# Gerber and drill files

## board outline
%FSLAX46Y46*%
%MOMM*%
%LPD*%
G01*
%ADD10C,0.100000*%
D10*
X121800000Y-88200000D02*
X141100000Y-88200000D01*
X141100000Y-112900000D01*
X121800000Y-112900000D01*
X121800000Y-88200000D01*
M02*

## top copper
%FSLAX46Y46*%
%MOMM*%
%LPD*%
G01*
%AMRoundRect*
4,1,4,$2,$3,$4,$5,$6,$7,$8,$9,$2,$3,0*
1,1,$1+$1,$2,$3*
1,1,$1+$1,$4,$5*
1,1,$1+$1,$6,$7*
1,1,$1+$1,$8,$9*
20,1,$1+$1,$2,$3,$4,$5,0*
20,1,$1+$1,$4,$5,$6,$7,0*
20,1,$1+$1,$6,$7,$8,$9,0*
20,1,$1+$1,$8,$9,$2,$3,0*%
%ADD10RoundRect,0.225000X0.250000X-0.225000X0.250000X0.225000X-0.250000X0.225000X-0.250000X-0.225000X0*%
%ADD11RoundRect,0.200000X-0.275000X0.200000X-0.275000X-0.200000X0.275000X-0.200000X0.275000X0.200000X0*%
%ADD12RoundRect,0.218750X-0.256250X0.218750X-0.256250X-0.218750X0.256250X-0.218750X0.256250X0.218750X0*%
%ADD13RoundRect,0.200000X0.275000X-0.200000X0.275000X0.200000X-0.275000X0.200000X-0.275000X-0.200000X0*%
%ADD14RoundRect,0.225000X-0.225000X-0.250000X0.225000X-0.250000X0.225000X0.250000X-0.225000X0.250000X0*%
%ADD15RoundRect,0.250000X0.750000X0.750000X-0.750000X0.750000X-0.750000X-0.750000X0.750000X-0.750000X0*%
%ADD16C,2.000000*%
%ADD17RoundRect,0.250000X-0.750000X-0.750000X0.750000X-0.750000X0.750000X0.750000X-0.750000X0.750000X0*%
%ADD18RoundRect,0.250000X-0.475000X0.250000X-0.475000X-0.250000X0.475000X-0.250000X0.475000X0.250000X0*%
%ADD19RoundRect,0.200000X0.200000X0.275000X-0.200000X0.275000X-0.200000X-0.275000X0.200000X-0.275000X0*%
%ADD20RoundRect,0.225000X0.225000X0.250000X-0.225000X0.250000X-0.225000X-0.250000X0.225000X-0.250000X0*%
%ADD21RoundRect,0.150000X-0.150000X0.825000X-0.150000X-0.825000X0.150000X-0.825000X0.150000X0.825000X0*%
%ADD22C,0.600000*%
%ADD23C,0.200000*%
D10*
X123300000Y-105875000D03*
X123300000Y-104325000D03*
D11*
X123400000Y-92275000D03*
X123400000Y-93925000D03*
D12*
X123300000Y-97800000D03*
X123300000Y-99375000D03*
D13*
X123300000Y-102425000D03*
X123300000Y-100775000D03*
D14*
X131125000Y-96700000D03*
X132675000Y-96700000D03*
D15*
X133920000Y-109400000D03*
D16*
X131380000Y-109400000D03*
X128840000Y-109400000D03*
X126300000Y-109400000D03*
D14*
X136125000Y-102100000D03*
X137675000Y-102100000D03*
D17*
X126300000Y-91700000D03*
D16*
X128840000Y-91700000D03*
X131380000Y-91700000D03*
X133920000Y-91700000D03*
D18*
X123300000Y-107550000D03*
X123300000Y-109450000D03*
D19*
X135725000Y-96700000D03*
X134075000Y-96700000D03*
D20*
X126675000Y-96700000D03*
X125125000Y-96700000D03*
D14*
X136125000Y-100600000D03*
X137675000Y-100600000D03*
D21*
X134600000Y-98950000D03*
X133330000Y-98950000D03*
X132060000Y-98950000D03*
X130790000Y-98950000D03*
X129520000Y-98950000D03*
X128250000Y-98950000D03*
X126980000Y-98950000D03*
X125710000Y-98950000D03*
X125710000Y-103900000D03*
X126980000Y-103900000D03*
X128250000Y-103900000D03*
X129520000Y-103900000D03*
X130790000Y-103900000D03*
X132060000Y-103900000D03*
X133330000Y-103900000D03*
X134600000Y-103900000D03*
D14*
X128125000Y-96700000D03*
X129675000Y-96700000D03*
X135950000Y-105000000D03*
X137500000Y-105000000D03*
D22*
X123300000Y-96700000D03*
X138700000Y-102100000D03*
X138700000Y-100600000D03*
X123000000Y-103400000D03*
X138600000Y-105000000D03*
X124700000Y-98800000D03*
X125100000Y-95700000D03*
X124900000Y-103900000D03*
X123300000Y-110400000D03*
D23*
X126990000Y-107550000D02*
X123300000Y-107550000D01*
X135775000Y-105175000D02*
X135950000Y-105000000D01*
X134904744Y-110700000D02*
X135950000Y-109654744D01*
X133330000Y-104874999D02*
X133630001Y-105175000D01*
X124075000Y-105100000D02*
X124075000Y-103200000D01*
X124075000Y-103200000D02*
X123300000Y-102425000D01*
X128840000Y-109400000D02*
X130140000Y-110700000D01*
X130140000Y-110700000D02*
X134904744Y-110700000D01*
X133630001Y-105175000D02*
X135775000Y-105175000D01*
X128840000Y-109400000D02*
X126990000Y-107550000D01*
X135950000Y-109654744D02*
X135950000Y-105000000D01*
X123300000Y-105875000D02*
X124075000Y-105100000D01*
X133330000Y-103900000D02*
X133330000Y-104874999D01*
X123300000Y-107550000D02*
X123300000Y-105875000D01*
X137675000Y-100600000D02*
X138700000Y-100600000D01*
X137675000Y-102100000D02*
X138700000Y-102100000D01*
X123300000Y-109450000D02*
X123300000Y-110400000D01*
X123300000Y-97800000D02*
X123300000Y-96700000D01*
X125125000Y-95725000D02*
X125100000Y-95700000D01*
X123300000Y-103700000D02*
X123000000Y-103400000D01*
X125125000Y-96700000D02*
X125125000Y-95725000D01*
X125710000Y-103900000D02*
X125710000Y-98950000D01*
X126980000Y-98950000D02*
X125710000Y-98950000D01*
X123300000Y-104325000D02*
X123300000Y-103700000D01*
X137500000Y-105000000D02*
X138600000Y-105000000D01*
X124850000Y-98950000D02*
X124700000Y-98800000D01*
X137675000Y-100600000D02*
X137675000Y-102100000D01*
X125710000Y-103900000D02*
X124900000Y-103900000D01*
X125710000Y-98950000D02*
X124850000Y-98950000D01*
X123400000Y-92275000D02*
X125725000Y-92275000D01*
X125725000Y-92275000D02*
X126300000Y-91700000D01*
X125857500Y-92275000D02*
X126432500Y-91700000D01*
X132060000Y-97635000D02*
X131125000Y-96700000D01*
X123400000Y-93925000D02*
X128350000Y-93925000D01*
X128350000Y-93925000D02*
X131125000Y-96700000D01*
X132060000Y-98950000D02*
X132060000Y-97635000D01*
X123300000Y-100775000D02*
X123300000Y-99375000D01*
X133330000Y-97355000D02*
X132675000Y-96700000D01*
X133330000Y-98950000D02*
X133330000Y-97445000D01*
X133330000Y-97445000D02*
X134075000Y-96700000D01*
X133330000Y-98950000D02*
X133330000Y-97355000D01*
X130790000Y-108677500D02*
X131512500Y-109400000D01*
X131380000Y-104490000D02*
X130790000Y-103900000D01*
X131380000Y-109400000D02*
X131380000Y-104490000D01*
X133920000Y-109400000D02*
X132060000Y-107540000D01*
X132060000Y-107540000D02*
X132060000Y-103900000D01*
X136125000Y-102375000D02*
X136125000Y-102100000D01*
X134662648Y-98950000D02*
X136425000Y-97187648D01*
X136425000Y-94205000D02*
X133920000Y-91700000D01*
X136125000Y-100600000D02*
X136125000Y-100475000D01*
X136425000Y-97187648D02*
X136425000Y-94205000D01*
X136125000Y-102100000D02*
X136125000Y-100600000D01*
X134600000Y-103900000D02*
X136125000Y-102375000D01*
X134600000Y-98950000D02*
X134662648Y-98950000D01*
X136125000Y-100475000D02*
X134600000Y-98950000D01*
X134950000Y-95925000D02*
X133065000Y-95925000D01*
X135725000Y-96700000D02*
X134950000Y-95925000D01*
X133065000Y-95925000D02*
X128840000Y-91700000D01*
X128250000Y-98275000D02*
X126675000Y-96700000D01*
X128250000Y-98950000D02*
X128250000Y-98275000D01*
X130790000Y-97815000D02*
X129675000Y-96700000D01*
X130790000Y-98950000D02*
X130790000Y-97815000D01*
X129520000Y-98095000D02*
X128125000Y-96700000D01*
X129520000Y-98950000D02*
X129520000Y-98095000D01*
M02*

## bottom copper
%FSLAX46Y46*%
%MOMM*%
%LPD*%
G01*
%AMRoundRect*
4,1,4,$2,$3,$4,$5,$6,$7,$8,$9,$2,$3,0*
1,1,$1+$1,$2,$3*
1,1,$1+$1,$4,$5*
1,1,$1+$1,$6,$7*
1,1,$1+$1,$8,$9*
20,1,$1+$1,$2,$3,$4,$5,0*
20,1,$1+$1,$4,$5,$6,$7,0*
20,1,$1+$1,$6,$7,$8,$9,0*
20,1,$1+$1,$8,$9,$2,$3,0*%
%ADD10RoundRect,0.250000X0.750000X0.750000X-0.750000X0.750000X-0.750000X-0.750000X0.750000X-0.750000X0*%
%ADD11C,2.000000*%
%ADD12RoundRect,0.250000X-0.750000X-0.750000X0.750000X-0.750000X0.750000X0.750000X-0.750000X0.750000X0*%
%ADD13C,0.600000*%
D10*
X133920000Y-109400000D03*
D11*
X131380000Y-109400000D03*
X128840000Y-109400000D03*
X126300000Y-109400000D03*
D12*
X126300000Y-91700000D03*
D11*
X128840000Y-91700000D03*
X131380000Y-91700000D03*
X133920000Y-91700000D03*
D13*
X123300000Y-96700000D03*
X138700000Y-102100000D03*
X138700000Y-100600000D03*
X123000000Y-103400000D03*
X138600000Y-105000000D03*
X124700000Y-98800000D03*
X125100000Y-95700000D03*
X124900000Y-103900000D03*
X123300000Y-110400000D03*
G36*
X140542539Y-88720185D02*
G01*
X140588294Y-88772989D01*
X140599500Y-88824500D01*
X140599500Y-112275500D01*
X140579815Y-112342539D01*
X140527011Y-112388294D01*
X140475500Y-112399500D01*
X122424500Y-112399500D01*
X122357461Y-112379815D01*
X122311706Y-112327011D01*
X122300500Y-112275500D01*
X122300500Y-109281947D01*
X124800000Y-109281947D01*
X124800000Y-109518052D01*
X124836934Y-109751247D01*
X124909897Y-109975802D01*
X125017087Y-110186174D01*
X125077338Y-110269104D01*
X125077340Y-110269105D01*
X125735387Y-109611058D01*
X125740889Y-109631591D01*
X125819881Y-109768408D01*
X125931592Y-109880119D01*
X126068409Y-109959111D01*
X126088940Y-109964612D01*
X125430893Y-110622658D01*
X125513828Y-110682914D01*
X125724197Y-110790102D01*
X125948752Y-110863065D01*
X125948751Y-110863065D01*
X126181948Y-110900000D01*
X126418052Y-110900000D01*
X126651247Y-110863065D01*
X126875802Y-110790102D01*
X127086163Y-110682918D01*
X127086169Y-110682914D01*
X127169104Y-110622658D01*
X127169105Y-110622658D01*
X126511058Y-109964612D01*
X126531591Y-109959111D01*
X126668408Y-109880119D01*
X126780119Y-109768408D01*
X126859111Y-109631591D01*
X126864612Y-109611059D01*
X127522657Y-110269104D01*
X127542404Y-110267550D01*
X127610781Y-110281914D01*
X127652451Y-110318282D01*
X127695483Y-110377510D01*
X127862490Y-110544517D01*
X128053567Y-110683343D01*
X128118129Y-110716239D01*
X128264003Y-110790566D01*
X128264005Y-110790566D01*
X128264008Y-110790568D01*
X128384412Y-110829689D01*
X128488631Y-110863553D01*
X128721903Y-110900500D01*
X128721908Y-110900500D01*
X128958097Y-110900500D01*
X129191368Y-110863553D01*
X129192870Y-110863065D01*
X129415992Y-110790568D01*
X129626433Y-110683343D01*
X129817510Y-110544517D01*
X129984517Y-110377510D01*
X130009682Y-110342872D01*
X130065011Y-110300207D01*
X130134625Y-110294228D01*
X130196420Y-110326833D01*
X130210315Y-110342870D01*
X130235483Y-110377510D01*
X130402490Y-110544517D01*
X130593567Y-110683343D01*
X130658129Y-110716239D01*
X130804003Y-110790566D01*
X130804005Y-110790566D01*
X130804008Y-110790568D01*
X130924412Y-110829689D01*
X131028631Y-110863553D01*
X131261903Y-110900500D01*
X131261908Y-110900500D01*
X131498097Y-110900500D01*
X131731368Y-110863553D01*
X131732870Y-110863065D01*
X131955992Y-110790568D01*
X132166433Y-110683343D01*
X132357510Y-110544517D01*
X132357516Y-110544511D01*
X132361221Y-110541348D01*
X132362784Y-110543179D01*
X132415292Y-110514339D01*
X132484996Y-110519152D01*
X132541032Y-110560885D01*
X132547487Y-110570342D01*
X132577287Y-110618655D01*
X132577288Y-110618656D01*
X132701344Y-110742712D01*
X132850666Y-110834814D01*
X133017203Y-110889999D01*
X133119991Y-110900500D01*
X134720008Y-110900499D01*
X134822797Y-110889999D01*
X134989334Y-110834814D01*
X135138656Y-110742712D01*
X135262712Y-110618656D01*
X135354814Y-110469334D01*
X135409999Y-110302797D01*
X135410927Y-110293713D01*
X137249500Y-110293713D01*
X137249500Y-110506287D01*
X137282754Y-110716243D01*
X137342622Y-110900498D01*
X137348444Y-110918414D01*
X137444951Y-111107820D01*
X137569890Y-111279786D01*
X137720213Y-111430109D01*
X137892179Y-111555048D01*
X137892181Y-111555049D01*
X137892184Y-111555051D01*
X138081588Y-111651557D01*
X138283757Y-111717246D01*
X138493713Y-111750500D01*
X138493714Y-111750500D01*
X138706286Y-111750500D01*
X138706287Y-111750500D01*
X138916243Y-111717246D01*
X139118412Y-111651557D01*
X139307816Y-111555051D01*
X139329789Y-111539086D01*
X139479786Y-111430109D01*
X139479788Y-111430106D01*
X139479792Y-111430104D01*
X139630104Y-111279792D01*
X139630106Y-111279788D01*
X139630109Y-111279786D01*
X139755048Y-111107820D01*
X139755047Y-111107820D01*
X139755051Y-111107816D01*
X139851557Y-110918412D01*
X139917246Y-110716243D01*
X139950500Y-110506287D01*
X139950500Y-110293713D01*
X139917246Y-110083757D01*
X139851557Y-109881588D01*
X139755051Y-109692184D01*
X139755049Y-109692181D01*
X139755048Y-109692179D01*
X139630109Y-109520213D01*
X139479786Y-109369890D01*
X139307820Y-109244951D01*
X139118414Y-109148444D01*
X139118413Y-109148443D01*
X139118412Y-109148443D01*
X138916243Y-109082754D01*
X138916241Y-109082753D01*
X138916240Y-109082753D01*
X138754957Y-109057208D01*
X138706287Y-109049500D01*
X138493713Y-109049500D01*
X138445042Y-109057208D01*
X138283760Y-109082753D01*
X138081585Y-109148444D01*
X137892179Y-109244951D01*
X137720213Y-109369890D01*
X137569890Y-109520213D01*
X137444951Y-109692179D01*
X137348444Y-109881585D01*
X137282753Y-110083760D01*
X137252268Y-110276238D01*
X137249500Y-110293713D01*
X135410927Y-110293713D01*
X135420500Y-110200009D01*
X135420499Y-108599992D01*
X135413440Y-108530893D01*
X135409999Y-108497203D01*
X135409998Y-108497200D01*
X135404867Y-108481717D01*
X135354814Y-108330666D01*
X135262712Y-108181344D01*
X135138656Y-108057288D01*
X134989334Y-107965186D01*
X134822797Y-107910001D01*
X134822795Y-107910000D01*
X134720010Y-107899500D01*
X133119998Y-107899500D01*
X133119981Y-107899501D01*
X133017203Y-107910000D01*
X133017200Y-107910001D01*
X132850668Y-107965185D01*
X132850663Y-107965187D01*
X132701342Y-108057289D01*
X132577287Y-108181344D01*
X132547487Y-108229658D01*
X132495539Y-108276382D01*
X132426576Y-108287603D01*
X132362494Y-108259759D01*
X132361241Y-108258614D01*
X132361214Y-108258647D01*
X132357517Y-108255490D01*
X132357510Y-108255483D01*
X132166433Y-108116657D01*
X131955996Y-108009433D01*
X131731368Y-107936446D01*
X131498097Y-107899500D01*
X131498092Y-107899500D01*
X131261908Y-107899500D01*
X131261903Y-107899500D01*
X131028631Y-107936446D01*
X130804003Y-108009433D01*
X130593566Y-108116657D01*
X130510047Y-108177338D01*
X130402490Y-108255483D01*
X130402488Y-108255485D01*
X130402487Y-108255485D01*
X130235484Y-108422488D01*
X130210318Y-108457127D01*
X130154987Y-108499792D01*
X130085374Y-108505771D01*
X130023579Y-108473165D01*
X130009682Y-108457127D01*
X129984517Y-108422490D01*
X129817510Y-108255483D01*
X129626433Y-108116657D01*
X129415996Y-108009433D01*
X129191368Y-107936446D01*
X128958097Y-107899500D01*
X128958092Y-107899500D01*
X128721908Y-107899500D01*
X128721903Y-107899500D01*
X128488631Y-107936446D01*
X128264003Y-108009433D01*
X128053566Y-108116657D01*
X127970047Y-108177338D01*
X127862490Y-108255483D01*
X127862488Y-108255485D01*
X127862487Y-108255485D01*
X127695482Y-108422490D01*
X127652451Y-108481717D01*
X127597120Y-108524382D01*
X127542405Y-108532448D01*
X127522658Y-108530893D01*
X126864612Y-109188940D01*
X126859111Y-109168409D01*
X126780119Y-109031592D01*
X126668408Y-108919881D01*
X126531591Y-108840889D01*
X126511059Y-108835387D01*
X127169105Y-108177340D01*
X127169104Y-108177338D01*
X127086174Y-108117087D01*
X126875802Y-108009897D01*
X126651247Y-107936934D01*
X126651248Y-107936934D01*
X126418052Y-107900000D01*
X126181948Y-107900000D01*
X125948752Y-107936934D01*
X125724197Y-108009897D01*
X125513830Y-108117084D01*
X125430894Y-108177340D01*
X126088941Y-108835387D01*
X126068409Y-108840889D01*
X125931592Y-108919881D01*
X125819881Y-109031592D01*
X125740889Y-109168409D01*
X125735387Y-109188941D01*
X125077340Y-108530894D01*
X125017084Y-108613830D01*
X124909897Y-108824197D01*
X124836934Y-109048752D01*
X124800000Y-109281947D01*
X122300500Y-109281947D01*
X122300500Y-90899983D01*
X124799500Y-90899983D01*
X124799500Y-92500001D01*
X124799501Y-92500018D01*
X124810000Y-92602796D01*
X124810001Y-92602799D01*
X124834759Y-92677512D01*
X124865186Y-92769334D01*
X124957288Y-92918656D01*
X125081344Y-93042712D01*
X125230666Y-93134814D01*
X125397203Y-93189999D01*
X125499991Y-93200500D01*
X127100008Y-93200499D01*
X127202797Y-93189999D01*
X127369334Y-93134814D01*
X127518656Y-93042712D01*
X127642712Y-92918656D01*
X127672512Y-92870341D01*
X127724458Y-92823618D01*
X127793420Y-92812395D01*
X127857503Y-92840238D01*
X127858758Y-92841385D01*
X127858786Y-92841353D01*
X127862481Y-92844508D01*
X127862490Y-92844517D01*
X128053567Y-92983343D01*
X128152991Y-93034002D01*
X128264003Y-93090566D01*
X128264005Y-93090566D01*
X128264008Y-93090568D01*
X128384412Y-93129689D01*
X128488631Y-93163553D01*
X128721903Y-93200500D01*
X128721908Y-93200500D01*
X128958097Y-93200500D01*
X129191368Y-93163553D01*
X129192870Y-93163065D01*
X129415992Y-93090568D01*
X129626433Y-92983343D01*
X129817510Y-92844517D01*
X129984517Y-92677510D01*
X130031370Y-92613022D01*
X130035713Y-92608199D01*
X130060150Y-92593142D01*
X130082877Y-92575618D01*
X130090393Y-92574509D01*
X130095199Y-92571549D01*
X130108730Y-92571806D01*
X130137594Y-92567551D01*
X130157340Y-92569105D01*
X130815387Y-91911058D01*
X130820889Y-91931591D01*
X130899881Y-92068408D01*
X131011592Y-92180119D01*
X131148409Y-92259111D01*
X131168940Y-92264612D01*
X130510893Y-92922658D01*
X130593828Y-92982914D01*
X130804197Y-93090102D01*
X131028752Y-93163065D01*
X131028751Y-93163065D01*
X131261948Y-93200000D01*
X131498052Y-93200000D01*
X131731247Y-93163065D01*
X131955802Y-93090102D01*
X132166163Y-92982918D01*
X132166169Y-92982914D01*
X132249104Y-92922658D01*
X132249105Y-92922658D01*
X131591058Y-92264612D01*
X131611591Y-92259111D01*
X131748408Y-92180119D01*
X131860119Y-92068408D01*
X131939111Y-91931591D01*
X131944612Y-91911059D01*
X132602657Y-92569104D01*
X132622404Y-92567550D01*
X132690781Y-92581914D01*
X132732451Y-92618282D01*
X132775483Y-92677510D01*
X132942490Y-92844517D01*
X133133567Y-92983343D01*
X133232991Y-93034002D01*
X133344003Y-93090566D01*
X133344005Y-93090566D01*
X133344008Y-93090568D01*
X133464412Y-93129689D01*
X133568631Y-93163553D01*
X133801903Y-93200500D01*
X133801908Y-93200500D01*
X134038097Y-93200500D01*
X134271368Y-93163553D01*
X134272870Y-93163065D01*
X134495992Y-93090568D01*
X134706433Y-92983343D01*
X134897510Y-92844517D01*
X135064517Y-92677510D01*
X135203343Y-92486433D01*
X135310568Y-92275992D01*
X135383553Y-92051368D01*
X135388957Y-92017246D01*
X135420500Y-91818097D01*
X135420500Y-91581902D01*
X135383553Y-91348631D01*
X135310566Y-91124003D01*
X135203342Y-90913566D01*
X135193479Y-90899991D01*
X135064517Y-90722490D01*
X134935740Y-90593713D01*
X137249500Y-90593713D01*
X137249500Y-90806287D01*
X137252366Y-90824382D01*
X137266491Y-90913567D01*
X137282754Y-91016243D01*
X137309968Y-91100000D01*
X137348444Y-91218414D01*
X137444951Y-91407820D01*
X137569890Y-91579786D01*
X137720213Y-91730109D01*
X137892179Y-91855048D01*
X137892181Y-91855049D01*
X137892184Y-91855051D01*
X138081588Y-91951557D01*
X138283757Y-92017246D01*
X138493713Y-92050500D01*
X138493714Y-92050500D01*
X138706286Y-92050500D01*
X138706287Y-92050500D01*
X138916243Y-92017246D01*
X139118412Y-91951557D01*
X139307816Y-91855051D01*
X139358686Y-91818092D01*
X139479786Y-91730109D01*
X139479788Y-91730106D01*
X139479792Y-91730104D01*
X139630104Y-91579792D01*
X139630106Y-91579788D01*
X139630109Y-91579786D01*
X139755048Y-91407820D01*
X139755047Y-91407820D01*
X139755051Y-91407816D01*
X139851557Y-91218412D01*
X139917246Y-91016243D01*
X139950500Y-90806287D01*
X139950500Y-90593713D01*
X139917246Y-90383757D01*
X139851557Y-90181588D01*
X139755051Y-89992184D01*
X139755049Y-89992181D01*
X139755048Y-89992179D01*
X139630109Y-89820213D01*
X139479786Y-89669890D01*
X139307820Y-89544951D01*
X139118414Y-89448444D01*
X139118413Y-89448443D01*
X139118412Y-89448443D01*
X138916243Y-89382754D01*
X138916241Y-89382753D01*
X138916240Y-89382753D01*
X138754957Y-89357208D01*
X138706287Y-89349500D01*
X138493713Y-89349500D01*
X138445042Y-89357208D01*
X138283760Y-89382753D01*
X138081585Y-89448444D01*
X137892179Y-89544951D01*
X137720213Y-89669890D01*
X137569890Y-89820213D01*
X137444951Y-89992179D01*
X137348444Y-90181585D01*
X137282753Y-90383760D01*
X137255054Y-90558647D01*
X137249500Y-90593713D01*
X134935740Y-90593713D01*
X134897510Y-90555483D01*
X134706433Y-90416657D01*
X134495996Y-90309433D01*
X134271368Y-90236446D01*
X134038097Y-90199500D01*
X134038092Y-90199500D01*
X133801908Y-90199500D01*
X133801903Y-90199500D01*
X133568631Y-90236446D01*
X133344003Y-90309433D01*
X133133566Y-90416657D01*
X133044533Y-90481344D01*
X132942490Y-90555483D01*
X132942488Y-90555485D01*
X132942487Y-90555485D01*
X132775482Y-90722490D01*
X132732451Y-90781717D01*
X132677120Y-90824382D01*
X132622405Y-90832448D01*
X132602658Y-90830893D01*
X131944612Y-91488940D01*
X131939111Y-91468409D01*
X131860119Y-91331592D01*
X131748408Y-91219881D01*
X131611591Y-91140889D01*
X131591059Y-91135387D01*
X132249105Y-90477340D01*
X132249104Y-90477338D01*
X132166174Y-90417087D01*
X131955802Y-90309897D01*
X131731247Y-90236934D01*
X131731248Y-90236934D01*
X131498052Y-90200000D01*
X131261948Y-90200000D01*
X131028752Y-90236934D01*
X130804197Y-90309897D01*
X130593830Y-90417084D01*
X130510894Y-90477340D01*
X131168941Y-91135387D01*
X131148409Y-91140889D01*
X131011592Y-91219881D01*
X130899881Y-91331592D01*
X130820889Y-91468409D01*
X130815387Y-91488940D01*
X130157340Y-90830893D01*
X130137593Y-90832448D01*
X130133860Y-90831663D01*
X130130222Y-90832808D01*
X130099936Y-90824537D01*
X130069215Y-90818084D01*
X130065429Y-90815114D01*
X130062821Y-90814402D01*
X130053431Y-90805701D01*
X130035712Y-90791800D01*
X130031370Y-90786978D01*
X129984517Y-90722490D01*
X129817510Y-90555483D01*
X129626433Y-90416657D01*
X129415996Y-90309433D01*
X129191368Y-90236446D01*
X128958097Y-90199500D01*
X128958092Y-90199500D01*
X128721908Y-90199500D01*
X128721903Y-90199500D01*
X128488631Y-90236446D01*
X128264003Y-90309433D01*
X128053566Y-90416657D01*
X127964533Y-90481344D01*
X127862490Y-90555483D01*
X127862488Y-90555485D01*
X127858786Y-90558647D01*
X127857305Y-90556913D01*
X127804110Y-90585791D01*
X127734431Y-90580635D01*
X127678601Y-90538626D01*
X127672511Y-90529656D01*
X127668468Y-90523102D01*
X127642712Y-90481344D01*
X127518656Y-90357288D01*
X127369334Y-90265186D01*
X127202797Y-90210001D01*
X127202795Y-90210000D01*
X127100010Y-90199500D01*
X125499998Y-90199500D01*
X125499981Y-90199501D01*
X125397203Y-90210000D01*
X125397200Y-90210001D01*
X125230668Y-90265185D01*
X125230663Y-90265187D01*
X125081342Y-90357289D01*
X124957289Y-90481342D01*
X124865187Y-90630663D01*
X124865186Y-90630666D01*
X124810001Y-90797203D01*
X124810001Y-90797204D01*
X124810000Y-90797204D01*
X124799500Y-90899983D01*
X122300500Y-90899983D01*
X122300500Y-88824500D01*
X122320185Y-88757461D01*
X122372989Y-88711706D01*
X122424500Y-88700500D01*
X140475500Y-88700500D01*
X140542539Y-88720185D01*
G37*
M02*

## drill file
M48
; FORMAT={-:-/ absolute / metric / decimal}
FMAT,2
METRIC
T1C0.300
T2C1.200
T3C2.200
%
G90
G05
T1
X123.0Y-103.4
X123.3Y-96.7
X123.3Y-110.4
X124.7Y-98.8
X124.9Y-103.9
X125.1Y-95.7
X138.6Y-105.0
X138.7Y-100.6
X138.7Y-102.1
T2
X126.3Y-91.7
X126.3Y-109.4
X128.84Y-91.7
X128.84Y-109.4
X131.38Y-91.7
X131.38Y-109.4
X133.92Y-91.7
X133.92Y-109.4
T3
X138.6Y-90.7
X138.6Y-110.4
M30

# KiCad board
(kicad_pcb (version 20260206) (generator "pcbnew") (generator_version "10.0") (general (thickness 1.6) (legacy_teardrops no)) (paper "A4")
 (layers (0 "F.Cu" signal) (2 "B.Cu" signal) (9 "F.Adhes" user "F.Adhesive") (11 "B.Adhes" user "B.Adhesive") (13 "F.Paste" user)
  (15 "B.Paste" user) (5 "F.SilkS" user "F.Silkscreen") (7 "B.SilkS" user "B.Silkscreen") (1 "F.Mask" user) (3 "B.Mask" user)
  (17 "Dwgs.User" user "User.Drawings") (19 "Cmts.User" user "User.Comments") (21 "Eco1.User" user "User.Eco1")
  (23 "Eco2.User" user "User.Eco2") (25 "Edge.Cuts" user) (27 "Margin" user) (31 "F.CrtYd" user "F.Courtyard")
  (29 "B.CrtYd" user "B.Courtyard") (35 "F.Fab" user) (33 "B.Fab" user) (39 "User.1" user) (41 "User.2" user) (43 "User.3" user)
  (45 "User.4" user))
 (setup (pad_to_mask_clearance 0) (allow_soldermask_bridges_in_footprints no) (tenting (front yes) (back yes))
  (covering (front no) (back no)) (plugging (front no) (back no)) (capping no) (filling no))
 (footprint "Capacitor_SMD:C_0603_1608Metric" (layer "F.Cu") (at 123.3 105.1 90)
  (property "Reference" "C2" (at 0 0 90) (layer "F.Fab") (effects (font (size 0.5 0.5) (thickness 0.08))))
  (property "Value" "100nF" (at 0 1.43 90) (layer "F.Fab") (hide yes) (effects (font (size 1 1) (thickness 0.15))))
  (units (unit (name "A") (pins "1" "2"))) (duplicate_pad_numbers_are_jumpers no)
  (pad "1" smd roundrect (at -0.775 0 90) (size 0.9 0.95) (layers "F.Cu" "F.Mask" "F.Paste") (roundrect_rratio 0.25) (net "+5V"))
  (pad "2" smd roundrect (at 0.775 0 90) (size 0.9 0.95) (layers "F.Cu" "F.Mask" "F.Paste") (roundrect_rratio 0.25) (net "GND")))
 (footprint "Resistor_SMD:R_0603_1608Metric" (layer "F.Cu") (at 123.4 93.1 -90)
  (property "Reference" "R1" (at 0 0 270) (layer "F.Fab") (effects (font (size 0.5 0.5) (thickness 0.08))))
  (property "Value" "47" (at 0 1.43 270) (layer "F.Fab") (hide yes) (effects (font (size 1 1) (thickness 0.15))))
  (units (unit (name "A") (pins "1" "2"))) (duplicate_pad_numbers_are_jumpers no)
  (pad "1" smd roundrect (at -0.825 0 270) (size 0.8 0.95) (layers "F.Cu" "F.Mask" "F.Paste") (roundrect_rratio 0.25) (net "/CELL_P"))
  (pad "2" smd roundrect (at 0.825 0 270) (size 0.8 0.95) (layers "F.Cu" "F.Mask" "F.Paste") (roundrect_rratio 0.25) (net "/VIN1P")))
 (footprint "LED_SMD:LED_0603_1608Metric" (layer "F.Cu") (at 123.3 98.5875 -90)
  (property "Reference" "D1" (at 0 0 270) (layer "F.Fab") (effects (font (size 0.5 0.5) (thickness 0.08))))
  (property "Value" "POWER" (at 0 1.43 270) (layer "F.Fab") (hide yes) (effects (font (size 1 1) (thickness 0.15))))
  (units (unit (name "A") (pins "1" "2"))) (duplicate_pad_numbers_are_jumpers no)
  (pad "1" smd roundrect (at -0.7875 0 270) (size 0.875 0.95) (layers "F.Cu" "F.Mask" "F.Paste") (roundrect_rratio 0.25) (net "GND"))
  (pad "2" smd roundrect (at 0.7875 0 270) (size 0.875 0.95) (layers "F.Cu" "F.Mask" "F.Paste") (roundrect_rratio 0.25) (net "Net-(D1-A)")))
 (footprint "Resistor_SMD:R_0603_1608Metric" (layer "F.Cu") (at 123.3 101.6 90)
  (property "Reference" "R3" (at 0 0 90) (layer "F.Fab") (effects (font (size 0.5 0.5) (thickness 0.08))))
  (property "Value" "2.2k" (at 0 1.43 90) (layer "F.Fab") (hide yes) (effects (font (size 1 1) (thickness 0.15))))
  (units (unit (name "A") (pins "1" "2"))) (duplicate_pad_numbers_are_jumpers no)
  (pad "1" smd roundrect (at -0.825 0 90) (size 0.8 0.95) (layers "F.Cu" "F.Mask" "F.Paste") (roundrect_rratio 0.25) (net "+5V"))
  (pad "2" smd roundrect (at 0.825 0 90) (size 0.8 0.95) (layers "F.Cu" "F.Mask" "F.Paste") (roundrect_rratio 0.25) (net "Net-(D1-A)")))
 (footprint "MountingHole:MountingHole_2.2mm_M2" (layer "F.Cu") (at 138.6 90.7)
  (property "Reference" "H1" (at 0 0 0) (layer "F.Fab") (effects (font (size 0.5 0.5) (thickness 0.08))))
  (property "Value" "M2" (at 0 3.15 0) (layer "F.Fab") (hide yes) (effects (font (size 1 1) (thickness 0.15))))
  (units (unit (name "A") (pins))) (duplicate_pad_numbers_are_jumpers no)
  (pad "" np_thru_hole circle (at 0 0) (size 2.2 2.2) (drill 2.2) (layers "*.Cu" "*.Mask")))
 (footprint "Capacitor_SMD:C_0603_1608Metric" (layer "F.Cu") (at 131.9 96.7)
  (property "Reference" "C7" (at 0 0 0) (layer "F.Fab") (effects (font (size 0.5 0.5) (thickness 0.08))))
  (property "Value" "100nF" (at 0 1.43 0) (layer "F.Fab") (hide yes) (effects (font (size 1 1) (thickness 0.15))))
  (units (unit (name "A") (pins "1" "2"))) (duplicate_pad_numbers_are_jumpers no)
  (pad "1" smd roundrect (at -0.775 0) (size 0.9 0.95) (layers "F.Cu" "F.Mask" "F.Paste") (roundrect_rratio 0.25) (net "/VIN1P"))
  (pad "2" smd roundrect (at 0.775 0) (size 0.9 0.95) (layers "F.Cu" "F.Mask" "F.Paste") (roundrect_rratio 0.25) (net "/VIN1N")))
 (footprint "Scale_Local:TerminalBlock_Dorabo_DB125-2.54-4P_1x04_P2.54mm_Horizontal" (layer "F.Cu") (at 133.92 109.4 180)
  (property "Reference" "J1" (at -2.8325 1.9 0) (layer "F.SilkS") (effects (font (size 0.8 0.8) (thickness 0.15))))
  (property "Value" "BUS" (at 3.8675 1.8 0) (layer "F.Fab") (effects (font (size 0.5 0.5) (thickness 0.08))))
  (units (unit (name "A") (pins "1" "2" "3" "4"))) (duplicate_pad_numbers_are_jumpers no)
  (pad "1" thru_hole roundrect (at 0 0 180) (size 2 2) (drill 1.2) (layers "*.Cu" "*.Mask") (remove_unused_layers no)
   (roundrect_rratio 0.125) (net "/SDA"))
  (pad "2" thru_hole circle (at 2.54 0 180) (size 2 2) (drill 1.2) (layers "*.Cu" "*.Mask") (remove_unused_layers no) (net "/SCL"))
  (pad "3" thru_hole circle (at 5.08 0 180) (size 2 2) (drill 1.2) (layers "*.Cu" "*.Mask") (remove_unused_layers no) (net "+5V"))
  (pad "4" thru_hole circle (at 7.62 0 180) (size 2 2) (drill 1.2) (layers "*.Cu" "*.Mask") (remove_unused_layers no) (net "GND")))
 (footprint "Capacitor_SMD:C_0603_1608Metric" (layer "F.Cu") (at 136.9 102.1)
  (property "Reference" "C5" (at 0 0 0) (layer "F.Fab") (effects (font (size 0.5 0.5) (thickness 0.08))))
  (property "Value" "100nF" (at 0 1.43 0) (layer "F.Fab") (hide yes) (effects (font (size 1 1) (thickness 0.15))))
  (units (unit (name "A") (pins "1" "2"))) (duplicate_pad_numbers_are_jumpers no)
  (pad "1" smd roundrect (at -0.775 0) (size 0.9 0.95) (layers "F.Cu" "F.Mask" "F.Paste") (roundrect_rratio 0.25) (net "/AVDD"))
  (pad "2" smd roundrect (at 0.775 0) (size 0.9 0.95) (layers "F.Cu" "F.Mask" "F.Paste") (roundrect_rratio 0.25) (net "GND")))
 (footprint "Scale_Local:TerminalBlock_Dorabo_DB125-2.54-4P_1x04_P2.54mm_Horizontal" (layer "F.Cu") (at 126.3 91.7)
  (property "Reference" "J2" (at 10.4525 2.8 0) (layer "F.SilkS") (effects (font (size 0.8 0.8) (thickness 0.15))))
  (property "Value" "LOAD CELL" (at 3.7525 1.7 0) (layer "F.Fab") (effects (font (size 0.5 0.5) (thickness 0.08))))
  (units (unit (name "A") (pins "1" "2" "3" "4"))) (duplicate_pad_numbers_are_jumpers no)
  (pad "1" thru_hole roundrect (at 0 0) (size 2 2) (drill 1.2) (layers "*.Cu" "*.Mask") (remove_unused_layers no) (roundrect_rratio 0.125)
   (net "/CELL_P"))
  (pad "2" thru_hole circle (at 2.54 0) (size 2 2) (drill 1.2) (layers "*.Cu" "*.Mask") (remove_unused_layers no) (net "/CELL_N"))
  (pad "3" thru_hole circle (at 5.08 0) (size 2 2) (drill 1.2) (layers "*.Cu" "*.Mask") (remove_unused_layers no) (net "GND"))
  (pad "4" thru_hole circle (at 7.62 0) (size 2 2) (drill 1.2) (layers "*.Cu" "*.Mask") (remove_unused_layers no) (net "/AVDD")))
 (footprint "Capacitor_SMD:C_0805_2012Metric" (layer "F.Cu") (at 123.3 108.5 -90)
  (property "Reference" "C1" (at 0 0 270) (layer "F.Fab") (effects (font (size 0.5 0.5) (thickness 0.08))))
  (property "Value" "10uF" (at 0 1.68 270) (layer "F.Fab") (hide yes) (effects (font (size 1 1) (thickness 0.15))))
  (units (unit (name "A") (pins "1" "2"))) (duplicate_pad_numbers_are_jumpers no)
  (pad "1" smd roundrect (at -0.95 0 270) (size 1 1.45) (layers "F.Cu" "F.Mask" "F.Paste") (roundrect_rratio 0.25) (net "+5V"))
  (pad "2" smd roundrect (at 0.95 0 270) (size 1 1.45) (layers "F.Cu" "F.Mask" "F.Paste") (roundrect_rratio 0.25) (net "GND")))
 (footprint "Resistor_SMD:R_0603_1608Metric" (layer "F.Cu") (at 134.9 96.7 180)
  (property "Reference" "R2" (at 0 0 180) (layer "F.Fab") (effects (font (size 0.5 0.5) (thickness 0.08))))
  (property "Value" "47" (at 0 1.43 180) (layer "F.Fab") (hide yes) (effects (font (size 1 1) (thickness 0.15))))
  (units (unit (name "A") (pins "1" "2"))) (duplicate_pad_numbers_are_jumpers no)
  (pad "1" smd roundrect (at -0.825 0 180) (size 0.8 0.95) (layers "F.Cu" "F.Mask" "F.Paste") (roundrect_rratio 0.25) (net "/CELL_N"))
  (pad "2" smd roundrect (at 0.825 0 180) (size 0.8 0.95) (layers "F.Cu" "F.Mask" "F.Paste") (roundrect_rratio 0.25) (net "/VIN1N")))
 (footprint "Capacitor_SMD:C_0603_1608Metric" (layer "F.Cu") (at 125.9 96.7 180)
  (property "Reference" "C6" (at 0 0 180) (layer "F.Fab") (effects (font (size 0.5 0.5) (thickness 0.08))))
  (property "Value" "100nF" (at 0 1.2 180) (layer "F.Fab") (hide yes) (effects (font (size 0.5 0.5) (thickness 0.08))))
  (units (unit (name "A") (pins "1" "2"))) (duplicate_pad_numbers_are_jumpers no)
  (pad "1" smd roundrect (at -0.775 0 180) (size 0.9 0.95) (layers "F.Cu" "F.Mask" "F.Paste") (roundrect_rratio 0.25) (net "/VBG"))
  (pad "2" smd roundrect (at 0.775 0 180) (size 0.9 0.95) (layers "F.Cu" "F.Mask" "F.Paste") (roundrect_rratio 0.25) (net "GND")))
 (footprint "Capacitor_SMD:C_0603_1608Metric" (layer "F.Cu") (at 136.9 100.6)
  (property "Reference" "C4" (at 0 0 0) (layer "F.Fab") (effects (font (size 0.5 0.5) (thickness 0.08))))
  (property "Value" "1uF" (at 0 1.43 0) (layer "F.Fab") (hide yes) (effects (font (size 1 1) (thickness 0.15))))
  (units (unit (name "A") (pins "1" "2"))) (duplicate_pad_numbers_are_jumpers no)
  (pad "1" smd roundrect (at -0.775 0) (size 0.9 0.95) (layers "F.Cu" "F.Mask" "F.Paste") (roundrect_rratio 0.25) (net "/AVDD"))
  (pad "2" smd roundrect (at 0.775 0) (size 0.9 0.95) (layers "F.Cu" "F.Mask" "F.Paste") (roundrect_rratio 0.25) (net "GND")))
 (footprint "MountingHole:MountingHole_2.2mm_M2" (layer "F.Cu") (at 138.6 110.4)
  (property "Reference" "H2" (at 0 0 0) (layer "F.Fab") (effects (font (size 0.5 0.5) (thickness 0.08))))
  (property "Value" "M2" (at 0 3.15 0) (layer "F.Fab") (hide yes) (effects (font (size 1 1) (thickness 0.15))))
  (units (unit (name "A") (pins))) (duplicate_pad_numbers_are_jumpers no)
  (pad "" np_thru_hole circle (at 0 0) (size 2.2 2.2) (drill 2.2) (layers "*.Cu" "*.Mask")))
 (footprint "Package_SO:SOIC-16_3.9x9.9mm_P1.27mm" (layer "F.Cu") (at 130.155 101.425 -90)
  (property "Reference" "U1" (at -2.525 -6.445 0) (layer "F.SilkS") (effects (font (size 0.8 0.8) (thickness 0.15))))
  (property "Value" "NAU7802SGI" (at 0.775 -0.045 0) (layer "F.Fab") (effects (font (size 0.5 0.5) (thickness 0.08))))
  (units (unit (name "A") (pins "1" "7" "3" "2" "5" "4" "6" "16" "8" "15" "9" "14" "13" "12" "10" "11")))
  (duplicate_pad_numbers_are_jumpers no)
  (pad "1" smd roundrect (at -2.475 -4.445 270) (size 1.95 0.6) (layers "F.Cu" "F.Mask" "F.Paste") (roundrect_rratio 0.25) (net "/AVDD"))
  (pad "2" smd roundrect (at -2.475 -3.175 270) (size 1.95 0.6) (layers "F.Cu" "F.Mask" "F.Paste") (roundrect_rratio 0.25) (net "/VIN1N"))
  (pad "3" smd roundrect (at -2.475 -1.905 270) (size 1.95 0.6) (layers "F.Cu" "F.Mask" "F.Paste") (roundrect_rratio 0.25) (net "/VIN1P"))
  (pad "4" smd roundrect (at -2.475 -0.635 270) (size 1.95 0.6) (layers "F.Cu" "F.Mask" "F.Paste") (roundrect_rratio 0.25) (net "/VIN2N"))
  (pad "5" smd roundrect (at -2.475 0.635 270) (size 1.95 0.6) (layers "F.Cu" "F.Mask" "F.Paste") (roundrect_rratio 0.25) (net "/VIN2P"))
  (pad "6" smd roundrect (at -2.475 1.905 270) (size 1.95 0.6) (layers "F.Cu" "F.Mask" "F.Paste") (roundrect_rratio 0.25) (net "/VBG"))
  (pad "7" smd roundrect (at -2.475 3.175 270) (size 1.95 0.6) (layers "F.Cu" "F.Mask" "F.Paste") (roundrect_rratio 0.25) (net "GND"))
  (pad "8" smd roundrect (at -2.475 4.445 270) (size 1.95 0.6) (layers "F.Cu" "F.Mask" "F.Paste") (roundrect_rratio 0.25) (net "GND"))
  (pad "9" smd roundrect (at 2.475 4.445 270) (size 1.95 0.6) (layers "F.Cu" "F.Mask" "F.Paste") (roundrect_rratio 0.25) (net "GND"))
  (pad "10" smd roundrect (at 2.475 3.175 270) (size 1.95 0.6) (layers "F.Cu" "F.Mask" "F.Paste") (roundrect_rratio 0.25)
   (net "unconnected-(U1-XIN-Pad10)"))
  (pad "11" smd roundrect (at 2.475 1.905 270) (size 1.95 0.6) (layers "F.Cu" "F.Mask" "F.Paste") (roundrect_rratio 0.25)
   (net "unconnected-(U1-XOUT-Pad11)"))
  (pad "12" smd roundrect (at 2.475 0.635 270) (size 1.95 0.6) (layers "F.Cu" "F.Mask" "F.Paste") (roundrect_rratio 0.25)
   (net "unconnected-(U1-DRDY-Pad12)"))
  (pad "13" smd roundrect (at 2.475 -0.635 270) (size 1.95 0.6) (layers "F.Cu" "F.Mask" "F.Paste") (roundrect_rratio 0.25) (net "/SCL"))
  (pad "14" smd roundrect (at 2.475 -1.905 270) (size 1.95 0.6) (layers "F.Cu" "F.Mask" "F.Paste") (roundrect_rratio 0.25) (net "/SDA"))
  (pad "15" smd roundrect (at 2.475 -3.175 270) (size 1.95 0.6) (layers "F.Cu" "F.Mask" "F.Paste") (roundrect_rratio 0.25) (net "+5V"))
  (pad "16" smd roundrect (at 2.475 -4.445 270) (size 1.95 0.6) (layers "F.Cu" "F.Mask" "F.Paste") (roundrect_rratio 0.25) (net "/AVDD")))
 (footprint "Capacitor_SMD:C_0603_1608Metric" (layer "F.Cu") (at 128.9 96.7)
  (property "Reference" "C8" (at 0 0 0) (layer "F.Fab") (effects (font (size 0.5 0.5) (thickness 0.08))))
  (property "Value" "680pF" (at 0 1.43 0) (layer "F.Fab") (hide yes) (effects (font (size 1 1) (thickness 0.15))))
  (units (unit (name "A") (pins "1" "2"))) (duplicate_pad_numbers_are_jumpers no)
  (pad "1" smd roundrect (at -0.775 0) (size 0.9 0.95) (layers "F.Cu" "F.Mask" "F.Paste") (roundrect_rratio 0.25) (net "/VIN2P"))
  (pad "2" smd roundrect (at 0.775 0) (size 0.9 0.95) (layers "F.Cu" "F.Mask" "F.Paste") (roundrect_rratio 0.25) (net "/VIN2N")))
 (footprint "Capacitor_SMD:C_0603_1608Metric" (layer "F.Cu") (at 136.725 105)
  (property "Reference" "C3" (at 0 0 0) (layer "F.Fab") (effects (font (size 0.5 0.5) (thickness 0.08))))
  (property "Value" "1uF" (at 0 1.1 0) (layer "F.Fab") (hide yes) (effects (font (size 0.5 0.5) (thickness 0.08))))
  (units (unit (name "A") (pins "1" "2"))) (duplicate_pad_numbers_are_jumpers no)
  (pad "1" smd roundrect (at -0.775 0) (size 0.9 0.95) (layers "F.Cu" "F.Mask" "F.Paste") (roundrect_rratio 0.25) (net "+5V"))
  (pad "2" smd roundrect (at 0.775 0) (size 0.9 0.95) (layers "F.Cu" "F.Mask" "F.Paste") (roundrect_rratio 0.25) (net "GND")))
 (gr_rect (start 121.8 88.2) (end 141.1 112.9) (stroke (width 0.1) (type default)) (fill no) (layer "Edge.Cuts"))
 (segment (start 126.99 107.55) (end 123.3 107.55) (width 0.2) (layer "F.Cu") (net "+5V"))
 (segment (start 135.775 105.175) (end 135.95 105) (width 0.2) (layer "F.Cu") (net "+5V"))
 (segment (start 134.904744 110.7) (end 135.95 109.654744) (width 0.2) (layer "F.Cu") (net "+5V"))
 (segment (start 133.33 104.874999) (end 133.630001 105.175) (width 0.2) (layer "F.Cu") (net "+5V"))
 (segment (start 124.075 105.1) (end 124.075 103.2) (width 0.2) (layer "F.Cu") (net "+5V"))
 (segment (start 124.075 103.2) (end 123.3 102.425) (width 0.2) (layer "F.Cu") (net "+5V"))
 (segment (start 128.84 109.4) (end 130.14 110.7) (width 0.2) (layer "F.Cu") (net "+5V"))
 (segment (start 130.14 110.7) (end 134.904744 110.7) (width 0.2) (layer "F.Cu") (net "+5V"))
 (segment (start 133.630001 105.175) (end 135.775 105.175) (width 0.2) (layer "F.Cu") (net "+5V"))
 (segment (start 128.84 109.4) (end 126.99 107.55) (width 0.2) (layer "F.Cu") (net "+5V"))
 (segment (start 135.95 109.654744) (end 135.95 105) (width 0.2) (layer "F.Cu") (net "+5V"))
 (segment (start 123.3 105.875) (end 124.075 105.1) (width 0.2) (layer "F.Cu") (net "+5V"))
 (segment (start 133.33 103.9) (end 133.33 104.874999) (width 0.2) (layer "F.Cu") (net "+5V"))
 (segment (start 123.3 107.55) (end 123.3 105.875) (width 0.2) (layer "F.Cu") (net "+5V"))
 (segment (start 137.675 100.6) (end 138.7 100.6) (width 0.2) (layer "F.Cu") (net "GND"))
 (segment (start 137.675 102.1) (end 138.7 102.1) (width 0.2) (layer "F.Cu") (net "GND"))
 (segment (start 123.3 109.45) (end 123.3 110.4) (width 0.2) (layer "F.Cu") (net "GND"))
 (segment (start 123.3 97.8) (end 123.3 96.7) (width 0.2) (layer "F.Cu") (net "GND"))
 (segment (start 125.125 95.725) (end 125.1 95.7) (width 0.2) (layer "F.Cu") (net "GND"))
 (segment (start 123.3 103.7) (end 123 103.4) (width 0.2) (layer "F.Cu") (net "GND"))
 (segment (start 125.125 96.7) (end 125.125 95.725) (width 0.2) (layer "F.Cu") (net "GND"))
 (segment (start 125.71 103.9) (end 125.71 98.95) (width 0.2) (layer "F.Cu") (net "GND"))
 (segment (start 126.98 98.95) (end 125.71 98.95) (width 0.2) (layer "F.Cu") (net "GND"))
 (segment (start 123.3 104.325) (end 123.3 103.7) (width 0.2) (layer "F.Cu") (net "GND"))
 (segment (start 137.5 105) (end 138.6 105) (width 0.2) (layer "F.Cu") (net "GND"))
 (segment (start 124.85 98.95) (end 124.7 98.8) (width 0.2) (layer "F.Cu") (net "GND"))
 (segment (start 137.675 100.6) (end 137.675 102.1) (width 0.2) (layer "F.Cu") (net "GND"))
 (segment (start 125.71 103.9) (end 124.9 103.9) (width 0.2) (layer "F.Cu") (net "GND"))
 (segment (start 125.71 98.95) (end 124.85 98.95) (width 0.2) (layer "F.Cu") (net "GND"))
 (via (at 123.3 96.7) (size 0.6) (drill 0.3) (layers "F.Cu" "B.Cu") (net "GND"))
 (via (at 138.7 102.1) (size 0.6) (drill 0.3) (layers "F.Cu" "B.Cu") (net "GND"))
 (via (at 138.7 100.6) (size 0.6) (drill 0.3) (layers "F.Cu" "B.Cu") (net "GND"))
 (via (at 123 103.4) (size 0.6) (drill 0.3) (layers "F.Cu" "B.Cu") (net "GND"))
 (via (at 138.6 105) (size 0.6) (drill 0.3) (layers "F.Cu" "B.Cu") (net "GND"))
 (via (at 124.7 98.8) (size 0.6) (drill 0.3) (layers "F.Cu" "B.Cu") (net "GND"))
 (via (at 125.1 95.7) (size 0.6) (drill 0.3) (layers "F.Cu" "B.Cu") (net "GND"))
 (via (at 124.9 103.9) (size 0.6) (drill 0.3) (layers "F.Cu" "B.Cu") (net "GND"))
 (via (at 123.3 110.4) (size 0.6) (drill 0.3) (layers "F.Cu" "B.Cu") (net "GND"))
 (segment (start 123.4 92.275) (end 125.725 92.275) (width 0.2) (layer "F.Cu") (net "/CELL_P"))
 (segment (start 125.725 92.275) (end 126.3 91.7) (width 0.2) (layer "F.Cu") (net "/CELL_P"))
 (segment (start 125.8575 92.275) (end 126.4325 91.7) (width 0.2) (layer "F.Cu") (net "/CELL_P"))
 (segment (start 132.06 97.635) (end 131.125 96.7) (width 0.2) (layer "F.Cu") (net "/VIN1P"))
 (segment (start 123.4 93.925) (end 128.35 93.925) (width 0.2) (layer "F.Cu") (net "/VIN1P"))
 (segment (start 128.35 93.925) (end 131.125 96.7) (width 0.2) (layer "F.Cu") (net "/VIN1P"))
 (segment (start 132.06 98.95) (end 132.06 97.635) (width 0.2) (layer "F.Cu") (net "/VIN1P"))
 (segment (start 123.3 100.775) (end 123.3 99.375) (width 0.2) (layer "F.Cu") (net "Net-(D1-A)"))
 (segment (start 133.33 97.355) (end 132.675 96.7) (width 0.2) (layer "F.Cu") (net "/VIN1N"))
 (segment (start 133.33 98.95) (end 133.33 97.445) (width 0.2) (layer "F.Cu") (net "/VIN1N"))
 (segment (start 133.33 97.445) (end 134.075 96.7) (width 0.2) (layer "F.Cu") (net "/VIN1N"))
 (segment (start 133.33 98.95) (end 133.33 97.355) (width 0.2) (layer "F.Cu") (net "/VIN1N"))
 (segment (start 130.79 108.6775) (end 131.5125 109.4) (width 0.2) (layer "F.Cu") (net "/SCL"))
 (segment (start 131.38 104.49) (end 130.79 103.9) (width 0.2) (layer "F.Cu") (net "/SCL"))
 (segment (start 131.38 109.4) (end 131.38 104.49) (width 0.2) (layer "F.Cu") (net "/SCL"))
 (segment (start 133.92 109.4) (end 132.06 107.54) (width 0.2) (layer "F.Cu") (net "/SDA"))
 (segment (start 132.06 107.54) (end 132.06 103.9) (width 0.2) (layer "F.Cu") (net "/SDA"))
 (segment (start 136.125 102.375) (end 136.125 102.1) (width 0.2) (layer "F.Cu") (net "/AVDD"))
 (segment (start 134.662648 98.95) (end 136.425 97.187648) (width 0.2) (layer "F.Cu") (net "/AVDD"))
 (segment (start 136.425 94.205) (end 133.92 91.7) (width 0.2) (layer "F.Cu") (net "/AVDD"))
 (segment (start 136.125 100.6) (end 136.125 100.475) (width 0.2) (layer "F.Cu") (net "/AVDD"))
 (segment (start 136.425 97.187648) (end 136.425 94.205) (width 0.2) (layer "F.Cu") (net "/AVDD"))
 (segment (start 136.125 102.1) (end 136.125 100.6) (width 0.2) (layer "F.Cu") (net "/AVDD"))
 (segment (start 134.6 103.9) (end 136.125 102.375) (width 0.2) (layer "F.Cu") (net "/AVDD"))
 (segment (start 134.6 98.95) (end 134.662648 98.95) (width 0.2) (layer "F.Cu") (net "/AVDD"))
 (segment (start 136.125 100.475) (end 134.6 98.95) (width 0.2) (layer "F.Cu") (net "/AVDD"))
 (segment (start 134.95 95.925) (end 133.065 95.925) (width 0.2) (layer "F.Cu") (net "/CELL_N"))
 (segment (start 135.725 96.7) (end 134.95 95.925) (width 0.2) (layer "F.Cu") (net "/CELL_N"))
 (segment (start 133.065 95.925) (end 128.84 91.7) (width 0.2) (layer "F.Cu") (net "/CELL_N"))
 (segment (start 128.25 98.275) (end 126.675 96.7) (width 0.2) (layer "F.Cu") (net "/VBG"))
 (segment (start 128.25 98.95) (end 128.25 98.275) (width 0.2) (layer "F.Cu") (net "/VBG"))
 (segment (start 130.79 97.815) (end 129.675 96.7) (width 0.2) (layer "F.Cu") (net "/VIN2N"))
 (segment (start 130.79 98.95) (end 130.79 97.815) (width 0.2) (layer "F.Cu") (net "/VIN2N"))
 (segment (start 129.52 98.095) (end 128.125 96.7) (width 0.2) (layer "F.Cu") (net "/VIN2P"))
 (segment (start 129.52 98.95) (end 129.52 98.095) (width 0.2) (layer "F.Cu") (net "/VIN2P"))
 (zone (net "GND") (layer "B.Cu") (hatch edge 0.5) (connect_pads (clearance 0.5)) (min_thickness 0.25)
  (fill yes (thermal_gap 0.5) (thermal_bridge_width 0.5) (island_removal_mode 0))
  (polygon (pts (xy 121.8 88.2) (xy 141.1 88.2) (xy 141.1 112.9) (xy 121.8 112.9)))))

